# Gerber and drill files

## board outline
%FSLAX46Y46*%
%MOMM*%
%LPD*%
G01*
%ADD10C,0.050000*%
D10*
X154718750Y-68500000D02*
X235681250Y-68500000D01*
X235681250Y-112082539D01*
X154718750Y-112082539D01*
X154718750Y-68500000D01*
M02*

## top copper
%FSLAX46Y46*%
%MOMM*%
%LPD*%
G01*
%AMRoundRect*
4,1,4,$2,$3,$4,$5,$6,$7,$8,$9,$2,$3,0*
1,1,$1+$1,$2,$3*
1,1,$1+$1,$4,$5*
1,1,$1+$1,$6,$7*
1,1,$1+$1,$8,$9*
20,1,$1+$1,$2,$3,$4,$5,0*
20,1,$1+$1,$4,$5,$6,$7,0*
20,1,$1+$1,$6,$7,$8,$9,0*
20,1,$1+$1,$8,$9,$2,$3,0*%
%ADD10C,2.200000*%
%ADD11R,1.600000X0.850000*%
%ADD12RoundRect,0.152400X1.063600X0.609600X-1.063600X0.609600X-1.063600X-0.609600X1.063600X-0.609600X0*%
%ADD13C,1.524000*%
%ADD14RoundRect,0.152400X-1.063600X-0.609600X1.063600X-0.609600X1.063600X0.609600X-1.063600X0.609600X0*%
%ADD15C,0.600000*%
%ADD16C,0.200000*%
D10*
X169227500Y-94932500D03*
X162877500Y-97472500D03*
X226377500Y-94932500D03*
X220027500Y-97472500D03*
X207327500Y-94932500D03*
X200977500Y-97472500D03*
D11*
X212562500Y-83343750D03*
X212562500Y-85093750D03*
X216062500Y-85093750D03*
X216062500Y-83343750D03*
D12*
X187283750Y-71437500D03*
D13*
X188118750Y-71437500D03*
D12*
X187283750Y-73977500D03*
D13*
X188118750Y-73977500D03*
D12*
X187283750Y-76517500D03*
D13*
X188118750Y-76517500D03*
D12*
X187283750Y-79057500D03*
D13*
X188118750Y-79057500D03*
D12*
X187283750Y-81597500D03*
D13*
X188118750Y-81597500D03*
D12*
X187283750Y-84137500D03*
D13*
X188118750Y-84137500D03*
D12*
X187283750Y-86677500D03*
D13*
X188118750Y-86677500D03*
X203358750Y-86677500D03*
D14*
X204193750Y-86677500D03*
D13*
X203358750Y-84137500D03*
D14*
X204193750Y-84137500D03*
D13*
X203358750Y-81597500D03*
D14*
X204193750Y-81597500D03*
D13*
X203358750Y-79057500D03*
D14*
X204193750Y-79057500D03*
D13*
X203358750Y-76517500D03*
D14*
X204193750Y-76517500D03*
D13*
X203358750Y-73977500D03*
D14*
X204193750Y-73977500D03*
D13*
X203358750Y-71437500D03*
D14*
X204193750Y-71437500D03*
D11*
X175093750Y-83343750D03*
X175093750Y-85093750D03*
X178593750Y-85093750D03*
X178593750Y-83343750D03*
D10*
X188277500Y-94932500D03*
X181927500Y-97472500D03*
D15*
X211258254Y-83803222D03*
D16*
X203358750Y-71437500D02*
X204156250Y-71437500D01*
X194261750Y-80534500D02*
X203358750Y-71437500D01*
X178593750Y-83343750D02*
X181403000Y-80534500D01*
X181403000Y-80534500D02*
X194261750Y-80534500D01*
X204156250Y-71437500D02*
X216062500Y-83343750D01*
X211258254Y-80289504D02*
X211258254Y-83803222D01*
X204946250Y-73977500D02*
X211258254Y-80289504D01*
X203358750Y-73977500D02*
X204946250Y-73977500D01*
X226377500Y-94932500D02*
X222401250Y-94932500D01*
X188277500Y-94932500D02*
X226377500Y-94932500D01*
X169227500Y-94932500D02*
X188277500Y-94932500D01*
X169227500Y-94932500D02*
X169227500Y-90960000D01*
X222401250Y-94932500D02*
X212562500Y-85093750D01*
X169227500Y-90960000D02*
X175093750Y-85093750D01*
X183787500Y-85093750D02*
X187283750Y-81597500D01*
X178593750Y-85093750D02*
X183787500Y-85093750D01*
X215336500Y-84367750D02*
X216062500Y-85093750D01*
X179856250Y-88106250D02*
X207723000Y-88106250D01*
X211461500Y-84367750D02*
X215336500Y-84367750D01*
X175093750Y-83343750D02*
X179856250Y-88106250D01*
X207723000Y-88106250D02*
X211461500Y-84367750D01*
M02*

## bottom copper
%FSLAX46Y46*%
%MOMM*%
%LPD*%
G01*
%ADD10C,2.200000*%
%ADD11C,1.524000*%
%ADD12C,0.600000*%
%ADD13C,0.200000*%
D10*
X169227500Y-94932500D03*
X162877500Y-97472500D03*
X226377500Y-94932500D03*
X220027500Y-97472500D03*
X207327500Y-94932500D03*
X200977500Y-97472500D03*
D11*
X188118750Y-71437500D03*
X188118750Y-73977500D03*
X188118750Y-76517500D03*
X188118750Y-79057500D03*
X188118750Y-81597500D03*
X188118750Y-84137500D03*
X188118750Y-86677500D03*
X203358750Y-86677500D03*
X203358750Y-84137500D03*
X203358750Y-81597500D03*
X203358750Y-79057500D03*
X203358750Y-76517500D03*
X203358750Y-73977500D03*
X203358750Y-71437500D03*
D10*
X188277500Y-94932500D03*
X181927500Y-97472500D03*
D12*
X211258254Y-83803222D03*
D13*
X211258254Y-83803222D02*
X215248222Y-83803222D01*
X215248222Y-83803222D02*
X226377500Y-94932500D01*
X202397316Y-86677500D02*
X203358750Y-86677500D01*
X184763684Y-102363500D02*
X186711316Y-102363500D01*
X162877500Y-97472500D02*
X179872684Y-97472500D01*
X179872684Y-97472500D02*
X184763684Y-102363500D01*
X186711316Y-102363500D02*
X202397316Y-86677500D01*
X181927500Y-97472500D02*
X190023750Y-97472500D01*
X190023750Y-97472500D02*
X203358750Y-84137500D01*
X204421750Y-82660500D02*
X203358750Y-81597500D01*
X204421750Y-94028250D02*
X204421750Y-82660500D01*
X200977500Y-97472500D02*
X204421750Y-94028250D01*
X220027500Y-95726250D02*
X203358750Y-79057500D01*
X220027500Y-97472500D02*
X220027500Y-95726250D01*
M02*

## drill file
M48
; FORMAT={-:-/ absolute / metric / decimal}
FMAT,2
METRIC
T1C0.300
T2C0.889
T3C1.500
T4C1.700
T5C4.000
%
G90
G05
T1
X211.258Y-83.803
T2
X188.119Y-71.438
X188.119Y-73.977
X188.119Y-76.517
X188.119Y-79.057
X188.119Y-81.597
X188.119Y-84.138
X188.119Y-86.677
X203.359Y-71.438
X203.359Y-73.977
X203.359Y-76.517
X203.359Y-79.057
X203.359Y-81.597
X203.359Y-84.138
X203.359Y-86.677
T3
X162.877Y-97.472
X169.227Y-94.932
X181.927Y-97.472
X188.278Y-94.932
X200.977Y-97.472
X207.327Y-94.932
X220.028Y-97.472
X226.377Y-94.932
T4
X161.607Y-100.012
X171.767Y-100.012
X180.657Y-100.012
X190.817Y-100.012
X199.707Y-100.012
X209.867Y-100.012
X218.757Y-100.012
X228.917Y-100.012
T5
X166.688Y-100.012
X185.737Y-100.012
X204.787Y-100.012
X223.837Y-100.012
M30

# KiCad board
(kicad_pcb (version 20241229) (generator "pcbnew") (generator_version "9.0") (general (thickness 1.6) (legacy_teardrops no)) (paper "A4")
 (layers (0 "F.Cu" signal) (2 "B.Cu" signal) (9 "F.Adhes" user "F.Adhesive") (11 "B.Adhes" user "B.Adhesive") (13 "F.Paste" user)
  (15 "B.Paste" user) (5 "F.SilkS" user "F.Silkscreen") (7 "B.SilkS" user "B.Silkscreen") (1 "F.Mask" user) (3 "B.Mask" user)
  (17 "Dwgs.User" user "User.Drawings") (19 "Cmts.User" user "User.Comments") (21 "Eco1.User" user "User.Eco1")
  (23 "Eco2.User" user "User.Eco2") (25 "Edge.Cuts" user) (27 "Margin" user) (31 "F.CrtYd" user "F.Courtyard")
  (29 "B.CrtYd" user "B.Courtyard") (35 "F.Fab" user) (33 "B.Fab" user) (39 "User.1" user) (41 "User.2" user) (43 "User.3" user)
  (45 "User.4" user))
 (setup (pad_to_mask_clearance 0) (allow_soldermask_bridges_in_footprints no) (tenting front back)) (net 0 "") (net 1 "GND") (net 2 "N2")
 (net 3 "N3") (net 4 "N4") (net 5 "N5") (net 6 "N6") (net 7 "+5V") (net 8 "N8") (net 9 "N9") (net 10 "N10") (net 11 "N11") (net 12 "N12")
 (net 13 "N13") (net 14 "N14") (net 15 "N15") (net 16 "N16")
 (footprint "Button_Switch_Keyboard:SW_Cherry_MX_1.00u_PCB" (layer "F.Cu") (at 169.2275 94.9325)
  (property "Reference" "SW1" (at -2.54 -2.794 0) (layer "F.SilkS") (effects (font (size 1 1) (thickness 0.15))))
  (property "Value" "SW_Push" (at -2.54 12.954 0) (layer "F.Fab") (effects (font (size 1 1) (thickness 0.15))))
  (pad "" np_thru_hole circle (at -7.62 5.08) (size 1.7 1.7) (drill 1.7) (layers "*.Cu" "*.Mask"))
  (pad "" np_thru_hole circle (at -2.54 5.08) (size 4 4) (drill 4) (layers "*.Cu" "*.Mask"))
  (pad "" np_thru_hole circle (at 2.54 5.08) (size 1.7 1.7) (drill 1.7) (layers "*.Cu" "*.Mask"))
  (pad "1" thru_hole circle (at 0 0) (size 2.2 2.2) (drill 1.5) (layers "*.Cu" "*.Mask") (remove_unused_layers no) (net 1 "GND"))
  (pad "2" thru_hole circle (at -6.35 2.54) (size 2.2 2.2) (drill 1.5) (layers "*.Cu" "*.Mask") (remove_unused_layers no) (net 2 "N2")))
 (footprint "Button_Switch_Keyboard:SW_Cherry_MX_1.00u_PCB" (layer "F.Cu") (at 226.3775 94.9325)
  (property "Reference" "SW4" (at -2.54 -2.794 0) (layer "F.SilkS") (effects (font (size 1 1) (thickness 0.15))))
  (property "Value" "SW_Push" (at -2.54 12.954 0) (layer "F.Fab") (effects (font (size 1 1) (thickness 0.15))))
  (pad "" np_thru_hole circle (at -7.62 5.08) (size 1.7 1.7) (drill 1.7) (layers "*.Cu" "*.Mask"))
  (pad "" np_thru_hole circle (at -2.54 5.08) (size 4 4) (drill 4) (layers "*.Cu" "*.Mask"))
  (pad "" np_thru_hole circle (at 2.54 5.08) (size 1.7 1.7) (drill 1.7) (layers "*.Cu" "*.Mask"))
  (pad "1" thru_hole circle (at 0 0) (size 2.2 2.2) (drill 1.5) (layers "*.Cu" "*.Mask") (remove_unused_layers no) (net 1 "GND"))
  (pad "2" thru_hole circle (at -6.35 2.54) (size 2.2 2.2) (drill 1.5) (layers "*.Cu" "*.Mask") (remove_unused_layers no) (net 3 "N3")))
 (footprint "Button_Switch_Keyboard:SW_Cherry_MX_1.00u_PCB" (layer "F.Cu") (at 207.3275 94.9325)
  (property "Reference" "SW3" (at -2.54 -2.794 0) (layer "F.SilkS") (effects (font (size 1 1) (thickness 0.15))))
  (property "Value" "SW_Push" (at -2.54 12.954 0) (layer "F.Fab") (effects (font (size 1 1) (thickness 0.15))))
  (pad "" np_thru_hole circle (at -7.62 5.08) (size 1.7 1.7) (drill 1.7) (layers "*.Cu" "*.Mask"))
  (pad "" np_thru_hole circle (at -2.54 5.08) (size 4 4) (drill 4) (layers "*.Cu" "*.Mask"))
  (pad "" np_thru_hole circle (at 2.54 5.08) (size 1.7 1.7) (drill 1.7) (layers "*.Cu" "*.Mask"))
  (pad "1" thru_hole circle (at 0 0) (size 2.2 2.2) (drill 1.5) (layers "*.Cu" "*.Mask") (remove_unused_layers no) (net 1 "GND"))
  (pad "2" thru_hole circle (at -6.35 2.54) (size 2.2 2.2) (drill 1.5) (layers "*.Cu" "*.Mask") (remove_unused_layers no) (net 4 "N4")))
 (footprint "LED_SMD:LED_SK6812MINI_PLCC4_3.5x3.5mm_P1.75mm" (layer "F.Cu") (at 214.3125 84.21875)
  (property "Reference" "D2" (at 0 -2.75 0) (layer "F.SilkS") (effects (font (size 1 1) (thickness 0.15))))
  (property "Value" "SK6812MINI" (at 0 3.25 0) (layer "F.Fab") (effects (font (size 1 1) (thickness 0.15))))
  (pad "1" smd rect (at -1.75 -0.875) (size 1.6 0.85) (layers "F.Cu" "F.Mask" "F.Paste") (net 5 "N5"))
  (pad "2" smd rect (at -1.75 0.875) (size 1.6 0.85) (layers "F.Cu" "F.Mask" "F.Paste") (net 1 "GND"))
  (pad "3" smd rect (at 1.75 0.875) (size 1.6 0.85) (layers "F.Cu" "F.Mask" "F.Paste") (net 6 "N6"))
  (pad "4" smd rect (at 1.75 -0.875) (size 1.6 0.85) (layers "F.Cu" "F.Mask" "F.Paste") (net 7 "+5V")))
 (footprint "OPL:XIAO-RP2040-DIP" (layer "F.Cu") (at 195.73875 79.0575)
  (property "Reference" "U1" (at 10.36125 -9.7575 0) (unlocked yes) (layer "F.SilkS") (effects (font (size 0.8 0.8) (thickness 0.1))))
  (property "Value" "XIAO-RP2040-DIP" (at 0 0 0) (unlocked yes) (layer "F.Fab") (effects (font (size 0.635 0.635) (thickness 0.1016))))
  (pad "1" smd roundrect (at -8.455 -7.62 180) (size 2.432 1.524) (layers "F.Cu" "F.Mask") (roundrect_rratio 0.1) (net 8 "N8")
   (thermal_bridge_angle 45))
  (pad "1" thru_hole circle (at -7.62 -7.62 180) (size 1.524 1.524) (drill 0.889) (layers "*.Cu" "*.Mask") (remove_unused_layers no)
   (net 8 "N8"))
  (pad "2" smd roundrect (at -8.455 -5.08 180) (size 2.432 1.524) (layers "F.Cu" "F.Mask") (roundrect_rratio 0.1) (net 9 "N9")
   (thermal_bridge_angle 45))
  (pad "2" thru_hole circle (at -7.62 -5.08 180) (size 1.524 1.524) (drill 0.889) (layers "*.Cu" "*.Mask") (remove_unused_layers no)
   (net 9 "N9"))
  (pad "3" smd roundrect (at -8.455 -2.54 180) (size 2.432 1.524) (layers "F.Cu" "F.Mask") (roundrect_rratio 0.1) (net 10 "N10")
   (thermal_bridge_angle 45))
  (pad "3" thru_hole circle (at -7.62 -2.54 180) (size 1.524 1.524) (drill 0.889) (layers "*.Cu" "*.Mask") (remove_unused_layers no)
   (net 10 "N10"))
  (pad "4" smd roundrect (at -8.455 0 180) (size 2.432 1.524) (layers "F.Cu" "F.Mask") (roundrect_rratio 0.1) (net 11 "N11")
   (thermal_bridge_angle 45))
  (pad "4" thru_hole circle (at -7.62 0 180) (size 1.524 1.524) (drill 0.889) (layers "*.Cu" "*.Mask") (remove_unused_layers no)
   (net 11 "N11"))
  (pad "5" smd roundrect (at -8.455 2.54 180) (size 2.432 1.524) (layers "F.Cu" "F.Mask") (roundrect_rratio 0.1) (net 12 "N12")
   (thermal_bridge_angle 45))
  (pad "5" thru_hole circle (at -7.62 2.54 180) (size 1.524 1.524) (drill 0.889) (layers "*.Cu" "*.Mask") (remove_unused_layers no)
   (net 12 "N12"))
  (pad "6" smd roundrect (at -8.455 5.08 180) (size 2.432 1.524) (layers "F.Cu" "F.Mask") (roundrect_rratio 0.1) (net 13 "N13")
   (thermal_bridge_angle 45))
  (pad "6" thru_hole circle (at -7.62 5.08 180) (size 1.524 1.524) (drill 0.889) (layers "*.Cu" "*.Mask") (remove_unused_layers no)
   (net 13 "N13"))
  (pad "7" smd roundrect (at -8.455 7.62 180) (size 2.432 1.524) (layers "F.Cu" "F.Mask") (roundrect_rratio 0.1) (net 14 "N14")
   (thermal_bridge_angle 45))
  (pad "7" thru_hole circle (at -7.62 7.62 180) (size 1.524 1.524) (drill 0.889) (layers "*.Cu" "*.Mask") (remove_unused_layers no)
   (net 14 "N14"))
  (pad "8" thru_hole circle (at 7.62 7.62) (size 1.524 1.524) (drill 0.889) (layers "*.Cu" "*.Mask") (remove_unused_layers no) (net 2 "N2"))
  (pad "8" smd roundrect (at 8.455 7.62) (size 2.432 1.524) (layers "F.Cu" "F.Mask") (roundrect_rratio 0.1) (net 2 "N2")
   (thermal_bridge_angle 45))
  (pad "9" thru_hole circle (at 7.62 5.08) (size 1.524 1.524) (drill 0.889) (layers "*.Cu" "*.Mask") (remove_unused_layers no)
   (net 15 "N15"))
  (pad "9" smd roundrect (at 8.455 5.08) (size 2.432 1.524) (layers "F.Cu" "F.Mask") (roundrect_rratio 0.1) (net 15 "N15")
   (thermal_bridge_angle 45))
  (pad "10" thru_hole circle (at 7.62 2.54) (size 1.524 1.524) (drill 0.889) (layers "*.Cu" "*.Mask") (remove_unused_layers no) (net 4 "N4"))
  (pad "10" smd roundrect (at 8.455 2.54) (size 2.432 1.524) (layers "F.Cu" "F.Mask") (roundrect_rratio 0.1) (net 4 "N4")
   (thermal_bridge_angle 45))
  (pad "11" thru_hole circle (at 7.62 0) (size 1.524 1.524) (drill 0.889) (layers "*.Cu" "*.Mask") (remove_unused_layers no) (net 3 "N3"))
  (pad "11" smd roundrect (at 8.455 0) (size 2.432 1.524) (layers "F.Cu" "F.Mask") (roundrect_rratio 0.1) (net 3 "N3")
   (thermal_bridge_angle 45))
  (pad "12" thru_hole circle (at 7.62 -2.54) (size 1.524 1.524) (drill 0.889) (layers "*.Cu" "*.Mask") (remove_unused_layers no)
   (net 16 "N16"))
  (pad "12" smd roundrect (at 8.455 -2.54) (size 2.432 1.524) (layers "F.Cu" "F.Mask") (roundrect_rratio 0.1) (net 16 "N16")
   (thermal_bridge_angle 45))
  (pad "13" thru_hole circle (at 7.62 -5.08) (size 1.524 1.524) (drill 0.889) (layers "*.Cu" "*.Mask") (remove_unused_layers no)
   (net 1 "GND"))
  (pad "13" smd roundrect (at 8.455 -5.08) (size 2.432 1.524) (layers "F.Cu" "F.Mask") (roundrect_rratio 0.1) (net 1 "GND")
   (thermal_bridge_angle 45))
  (pad "14" thru_hole circle (at 7.62 -7.62) (size 1.524 1.524) (drill 0.889) (layers "*.Cu" "*.Mask") (remove_unused_layers no)
   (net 7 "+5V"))
  (pad "14" smd roundrect (at 8.455 -7.62) (size 2.432 1.524) (layers "F.Cu" "F.Mask") (roundrect_rratio 0.1) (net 7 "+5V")
   (thermal_bridge_angle 45)))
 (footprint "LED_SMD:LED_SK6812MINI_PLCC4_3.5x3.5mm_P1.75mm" (layer "F.Cu") (at 176.84375 84.21875)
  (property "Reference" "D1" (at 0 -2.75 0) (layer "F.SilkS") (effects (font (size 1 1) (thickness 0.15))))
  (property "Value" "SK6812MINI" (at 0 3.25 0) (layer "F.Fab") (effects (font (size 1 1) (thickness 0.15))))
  (pad "1" smd rect (at -1.75 -0.875) (size 1.6 0.85) (layers "F.Cu" "F.Mask" "F.Paste") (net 6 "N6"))
  (pad "2" smd rect (at -1.75 0.875) (size 1.6 0.85) (layers "F.Cu" "F.Mask" "F.Paste") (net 1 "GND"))
  (pad "3" smd rect (at 1.75 0.875) (size 1.6 0.85) (layers "F.Cu" "F.Mask" "F.Paste") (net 12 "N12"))
  (pad "4" smd rect (at 1.75 -0.875) (size 1.6 0.85) (layers "F.Cu" "F.Mask" "F.Paste") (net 7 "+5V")))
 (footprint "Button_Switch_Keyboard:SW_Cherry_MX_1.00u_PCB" (layer "F.Cu") (at 188.2775 94.9325)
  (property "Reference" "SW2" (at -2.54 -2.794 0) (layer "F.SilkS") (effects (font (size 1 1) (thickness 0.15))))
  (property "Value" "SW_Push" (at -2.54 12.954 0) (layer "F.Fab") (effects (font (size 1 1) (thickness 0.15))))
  (pad "" np_thru_hole circle (at -7.62 5.08) (size 1.7 1.7) (drill 1.7) (layers "*.Cu" "*.Mask"))
  (pad "" np_thru_hole circle (at -2.54 5.08) (size 4 4) (drill 4) (layers "*.Cu" "*.Mask"))
  (pad "" np_thru_hole circle (at 2.54 5.08) (size 1.7 1.7) (drill 1.7) (layers "*.Cu" "*.Mask"))
  (pad "1" thru_hole circle (at 0 0) (size 2.2 2.2) (drill 1.5) (layers "*.Cu" "*.Mask") (remove_unused_layers no) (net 1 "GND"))
  (pad "2" thru_hole circle (at -6.35 2.54) (size 2.2 2.2) (drill 1.5) (layers "*.Cu" "*.Mask") (remove_unused_layers no) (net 15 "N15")))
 (gr_rect (start 154.71875 68.5) (end 235.68125 112.082539) (stroke (width 0.05) (type default)) (fill no) (layer "Edge.Cuts"))
 (segment (start 203.35875 71.4375) (end 204.15625 71.4375) (width 0.2) (layer "F.Cu") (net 7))
 (segment (start 194.26175 80.5345) (end 203.35875 71.4375) (width 0.2) (layer "F.Cu") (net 7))
 (segment (start 178.59375 83.34375) (end 181.403 80.5345) (width 0.2) (layer "F.Cu") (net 7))
 (segment (start 181.403 80.5345) (end 194.26175 80.5345) (width 0.2) (layer "F.Cu") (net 7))
 (segment (start 204.15625 71.4375) (end 216.0625 83.34375) (width 0.2) (layer "F.Cu") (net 7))
 (segment (start 211.258254 80.289504) (end 211.258254 83.803222) (width 0.2) (layer "F.Cu") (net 1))
 (segment (start 204.94625 73.9775) (end 211.258254 80.289504) (width 0.2) (layer "F.Cu") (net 1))
 (segment (start 203.35875 73.9775) (end 204.94625 73.9775) (width 0.2) (layer "F.Cu") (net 1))
 (segment (start 226.3775 94.9325) (end 222.40125 94.9325) (width 0.2) (layer "F.Cu") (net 1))
 (segment (start 188.2775 94.9325) (end 226.3775 94.9325) (width 0.2) (layer "F.Cu") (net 1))
 (segment (start 169.2275 94.9325) (end 188.2775 94.9325) (width 0.2) (layer "F.Cu") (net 1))
 (segment (start 169.2275 94.9325) (end 169.2275 90.96) (width 0.2) (layer "F.Cu") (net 1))
 (segment (start 222.40125 94.9325) (end 212.5625 85.09375) (width 0.2) (layer "F.Cu") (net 1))
 (segment (start 169.2275 90.96) (end 175.09375 85.09375) (width 0.2) (layer "F.Cu") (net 1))
 (via (at 211.258254 83.803222) (size 0.6) (drill 0.3) (layers "F.Cu" "B.Cu") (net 1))
 (segment (start 211.258254 83.803222) (end 215.248222 83.803222) (width 0.2) (layer "B.Cu") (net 1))
 (segment (start 215.248222 83.803222) (end 226.3775 94.9325) (width 0.2) (layer "B.Cu") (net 1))
 (segment (start 183.7875 85.09375) (end 187.28375 81.5975) (width 0.2) (layer "F.Cu") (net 12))
 (segment (start 178.59375 85.09375) (end 183.7875 85.09375) (width 0.2) (layer "F.Cu") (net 12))
 (segment (start 215.3365 84.36775) (end 216.0625 85.09375) (width 0.2) (layer "F.Cu") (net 6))
 (segment (start 179.85625 88.10625) (end 207.723 88.10625) (width 0.2) (layer "F.Cu") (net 6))
 (segment (start 211.4615 84.36775) (end 215.3365 84.36775) (width 0.2) (layer "F.Cu") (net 6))
 (segment (start 175.09375 83.34375) (end 179.85625 88.10625) (width 0.2) (layer "F.Cu") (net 6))
 (segment (start 207.723 88.10625) (end 211.4615 84.36775) (width 0.2) (layer "F.Cu") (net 6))
 (segment (start 202.397316 86.6775) (end 203.35875 86.6775) (width 0.2) (layer "B.Cu") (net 2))
 (segment (start 184.763684 102.3635) (end 186.711316 102.3635) (width 0.2) (layer "B.Cu") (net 2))
 (segment (start 162.8775 97.4725) (end 179.872684 97.4725) (width 0.2) (layer "B.Cu") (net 2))
 (segment (start 179.872684 97.4725) (end 184.763684 102.3635) (width 0.2) (layer "B.Cu") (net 2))
 (segment (start 186.711316 102.3635) (end 202.397316 86.6775) (width 0.2) (layer "B.Cu") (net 2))
 (segment (start 181.9275 97.4725) (end 190.02375 97.4725) (width 0.2) (layer "B.Cu") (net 15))
 (segment (start 190.02375 97.4725) (end 203.35875 84.1375) (width 0.2) (layer "B.Cu") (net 15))
 (segment (start 204.42175 82.6605) (end 203.35875 81.5975) (width 0.2) (layer "B.Cu") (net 4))
 (segment (start 204.42175 94.02825) (end 204.42175 82.6605) (width 0.2) (layer "B.Cu") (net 4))
 (segment (start 200.9775 97.4725) (end 204.42175 94.02825) (width 0.2) (layer "B.Cu") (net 4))
 (segment (start 220.0275 95.72625) (end 203.35875 79.0575) (width 0.2) (layer "B.Cu") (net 3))
 (segment (start 220.0275 97.4725) (end 220.0275 95.72625) (width 0.2) (layer "B.Cu") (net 3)))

